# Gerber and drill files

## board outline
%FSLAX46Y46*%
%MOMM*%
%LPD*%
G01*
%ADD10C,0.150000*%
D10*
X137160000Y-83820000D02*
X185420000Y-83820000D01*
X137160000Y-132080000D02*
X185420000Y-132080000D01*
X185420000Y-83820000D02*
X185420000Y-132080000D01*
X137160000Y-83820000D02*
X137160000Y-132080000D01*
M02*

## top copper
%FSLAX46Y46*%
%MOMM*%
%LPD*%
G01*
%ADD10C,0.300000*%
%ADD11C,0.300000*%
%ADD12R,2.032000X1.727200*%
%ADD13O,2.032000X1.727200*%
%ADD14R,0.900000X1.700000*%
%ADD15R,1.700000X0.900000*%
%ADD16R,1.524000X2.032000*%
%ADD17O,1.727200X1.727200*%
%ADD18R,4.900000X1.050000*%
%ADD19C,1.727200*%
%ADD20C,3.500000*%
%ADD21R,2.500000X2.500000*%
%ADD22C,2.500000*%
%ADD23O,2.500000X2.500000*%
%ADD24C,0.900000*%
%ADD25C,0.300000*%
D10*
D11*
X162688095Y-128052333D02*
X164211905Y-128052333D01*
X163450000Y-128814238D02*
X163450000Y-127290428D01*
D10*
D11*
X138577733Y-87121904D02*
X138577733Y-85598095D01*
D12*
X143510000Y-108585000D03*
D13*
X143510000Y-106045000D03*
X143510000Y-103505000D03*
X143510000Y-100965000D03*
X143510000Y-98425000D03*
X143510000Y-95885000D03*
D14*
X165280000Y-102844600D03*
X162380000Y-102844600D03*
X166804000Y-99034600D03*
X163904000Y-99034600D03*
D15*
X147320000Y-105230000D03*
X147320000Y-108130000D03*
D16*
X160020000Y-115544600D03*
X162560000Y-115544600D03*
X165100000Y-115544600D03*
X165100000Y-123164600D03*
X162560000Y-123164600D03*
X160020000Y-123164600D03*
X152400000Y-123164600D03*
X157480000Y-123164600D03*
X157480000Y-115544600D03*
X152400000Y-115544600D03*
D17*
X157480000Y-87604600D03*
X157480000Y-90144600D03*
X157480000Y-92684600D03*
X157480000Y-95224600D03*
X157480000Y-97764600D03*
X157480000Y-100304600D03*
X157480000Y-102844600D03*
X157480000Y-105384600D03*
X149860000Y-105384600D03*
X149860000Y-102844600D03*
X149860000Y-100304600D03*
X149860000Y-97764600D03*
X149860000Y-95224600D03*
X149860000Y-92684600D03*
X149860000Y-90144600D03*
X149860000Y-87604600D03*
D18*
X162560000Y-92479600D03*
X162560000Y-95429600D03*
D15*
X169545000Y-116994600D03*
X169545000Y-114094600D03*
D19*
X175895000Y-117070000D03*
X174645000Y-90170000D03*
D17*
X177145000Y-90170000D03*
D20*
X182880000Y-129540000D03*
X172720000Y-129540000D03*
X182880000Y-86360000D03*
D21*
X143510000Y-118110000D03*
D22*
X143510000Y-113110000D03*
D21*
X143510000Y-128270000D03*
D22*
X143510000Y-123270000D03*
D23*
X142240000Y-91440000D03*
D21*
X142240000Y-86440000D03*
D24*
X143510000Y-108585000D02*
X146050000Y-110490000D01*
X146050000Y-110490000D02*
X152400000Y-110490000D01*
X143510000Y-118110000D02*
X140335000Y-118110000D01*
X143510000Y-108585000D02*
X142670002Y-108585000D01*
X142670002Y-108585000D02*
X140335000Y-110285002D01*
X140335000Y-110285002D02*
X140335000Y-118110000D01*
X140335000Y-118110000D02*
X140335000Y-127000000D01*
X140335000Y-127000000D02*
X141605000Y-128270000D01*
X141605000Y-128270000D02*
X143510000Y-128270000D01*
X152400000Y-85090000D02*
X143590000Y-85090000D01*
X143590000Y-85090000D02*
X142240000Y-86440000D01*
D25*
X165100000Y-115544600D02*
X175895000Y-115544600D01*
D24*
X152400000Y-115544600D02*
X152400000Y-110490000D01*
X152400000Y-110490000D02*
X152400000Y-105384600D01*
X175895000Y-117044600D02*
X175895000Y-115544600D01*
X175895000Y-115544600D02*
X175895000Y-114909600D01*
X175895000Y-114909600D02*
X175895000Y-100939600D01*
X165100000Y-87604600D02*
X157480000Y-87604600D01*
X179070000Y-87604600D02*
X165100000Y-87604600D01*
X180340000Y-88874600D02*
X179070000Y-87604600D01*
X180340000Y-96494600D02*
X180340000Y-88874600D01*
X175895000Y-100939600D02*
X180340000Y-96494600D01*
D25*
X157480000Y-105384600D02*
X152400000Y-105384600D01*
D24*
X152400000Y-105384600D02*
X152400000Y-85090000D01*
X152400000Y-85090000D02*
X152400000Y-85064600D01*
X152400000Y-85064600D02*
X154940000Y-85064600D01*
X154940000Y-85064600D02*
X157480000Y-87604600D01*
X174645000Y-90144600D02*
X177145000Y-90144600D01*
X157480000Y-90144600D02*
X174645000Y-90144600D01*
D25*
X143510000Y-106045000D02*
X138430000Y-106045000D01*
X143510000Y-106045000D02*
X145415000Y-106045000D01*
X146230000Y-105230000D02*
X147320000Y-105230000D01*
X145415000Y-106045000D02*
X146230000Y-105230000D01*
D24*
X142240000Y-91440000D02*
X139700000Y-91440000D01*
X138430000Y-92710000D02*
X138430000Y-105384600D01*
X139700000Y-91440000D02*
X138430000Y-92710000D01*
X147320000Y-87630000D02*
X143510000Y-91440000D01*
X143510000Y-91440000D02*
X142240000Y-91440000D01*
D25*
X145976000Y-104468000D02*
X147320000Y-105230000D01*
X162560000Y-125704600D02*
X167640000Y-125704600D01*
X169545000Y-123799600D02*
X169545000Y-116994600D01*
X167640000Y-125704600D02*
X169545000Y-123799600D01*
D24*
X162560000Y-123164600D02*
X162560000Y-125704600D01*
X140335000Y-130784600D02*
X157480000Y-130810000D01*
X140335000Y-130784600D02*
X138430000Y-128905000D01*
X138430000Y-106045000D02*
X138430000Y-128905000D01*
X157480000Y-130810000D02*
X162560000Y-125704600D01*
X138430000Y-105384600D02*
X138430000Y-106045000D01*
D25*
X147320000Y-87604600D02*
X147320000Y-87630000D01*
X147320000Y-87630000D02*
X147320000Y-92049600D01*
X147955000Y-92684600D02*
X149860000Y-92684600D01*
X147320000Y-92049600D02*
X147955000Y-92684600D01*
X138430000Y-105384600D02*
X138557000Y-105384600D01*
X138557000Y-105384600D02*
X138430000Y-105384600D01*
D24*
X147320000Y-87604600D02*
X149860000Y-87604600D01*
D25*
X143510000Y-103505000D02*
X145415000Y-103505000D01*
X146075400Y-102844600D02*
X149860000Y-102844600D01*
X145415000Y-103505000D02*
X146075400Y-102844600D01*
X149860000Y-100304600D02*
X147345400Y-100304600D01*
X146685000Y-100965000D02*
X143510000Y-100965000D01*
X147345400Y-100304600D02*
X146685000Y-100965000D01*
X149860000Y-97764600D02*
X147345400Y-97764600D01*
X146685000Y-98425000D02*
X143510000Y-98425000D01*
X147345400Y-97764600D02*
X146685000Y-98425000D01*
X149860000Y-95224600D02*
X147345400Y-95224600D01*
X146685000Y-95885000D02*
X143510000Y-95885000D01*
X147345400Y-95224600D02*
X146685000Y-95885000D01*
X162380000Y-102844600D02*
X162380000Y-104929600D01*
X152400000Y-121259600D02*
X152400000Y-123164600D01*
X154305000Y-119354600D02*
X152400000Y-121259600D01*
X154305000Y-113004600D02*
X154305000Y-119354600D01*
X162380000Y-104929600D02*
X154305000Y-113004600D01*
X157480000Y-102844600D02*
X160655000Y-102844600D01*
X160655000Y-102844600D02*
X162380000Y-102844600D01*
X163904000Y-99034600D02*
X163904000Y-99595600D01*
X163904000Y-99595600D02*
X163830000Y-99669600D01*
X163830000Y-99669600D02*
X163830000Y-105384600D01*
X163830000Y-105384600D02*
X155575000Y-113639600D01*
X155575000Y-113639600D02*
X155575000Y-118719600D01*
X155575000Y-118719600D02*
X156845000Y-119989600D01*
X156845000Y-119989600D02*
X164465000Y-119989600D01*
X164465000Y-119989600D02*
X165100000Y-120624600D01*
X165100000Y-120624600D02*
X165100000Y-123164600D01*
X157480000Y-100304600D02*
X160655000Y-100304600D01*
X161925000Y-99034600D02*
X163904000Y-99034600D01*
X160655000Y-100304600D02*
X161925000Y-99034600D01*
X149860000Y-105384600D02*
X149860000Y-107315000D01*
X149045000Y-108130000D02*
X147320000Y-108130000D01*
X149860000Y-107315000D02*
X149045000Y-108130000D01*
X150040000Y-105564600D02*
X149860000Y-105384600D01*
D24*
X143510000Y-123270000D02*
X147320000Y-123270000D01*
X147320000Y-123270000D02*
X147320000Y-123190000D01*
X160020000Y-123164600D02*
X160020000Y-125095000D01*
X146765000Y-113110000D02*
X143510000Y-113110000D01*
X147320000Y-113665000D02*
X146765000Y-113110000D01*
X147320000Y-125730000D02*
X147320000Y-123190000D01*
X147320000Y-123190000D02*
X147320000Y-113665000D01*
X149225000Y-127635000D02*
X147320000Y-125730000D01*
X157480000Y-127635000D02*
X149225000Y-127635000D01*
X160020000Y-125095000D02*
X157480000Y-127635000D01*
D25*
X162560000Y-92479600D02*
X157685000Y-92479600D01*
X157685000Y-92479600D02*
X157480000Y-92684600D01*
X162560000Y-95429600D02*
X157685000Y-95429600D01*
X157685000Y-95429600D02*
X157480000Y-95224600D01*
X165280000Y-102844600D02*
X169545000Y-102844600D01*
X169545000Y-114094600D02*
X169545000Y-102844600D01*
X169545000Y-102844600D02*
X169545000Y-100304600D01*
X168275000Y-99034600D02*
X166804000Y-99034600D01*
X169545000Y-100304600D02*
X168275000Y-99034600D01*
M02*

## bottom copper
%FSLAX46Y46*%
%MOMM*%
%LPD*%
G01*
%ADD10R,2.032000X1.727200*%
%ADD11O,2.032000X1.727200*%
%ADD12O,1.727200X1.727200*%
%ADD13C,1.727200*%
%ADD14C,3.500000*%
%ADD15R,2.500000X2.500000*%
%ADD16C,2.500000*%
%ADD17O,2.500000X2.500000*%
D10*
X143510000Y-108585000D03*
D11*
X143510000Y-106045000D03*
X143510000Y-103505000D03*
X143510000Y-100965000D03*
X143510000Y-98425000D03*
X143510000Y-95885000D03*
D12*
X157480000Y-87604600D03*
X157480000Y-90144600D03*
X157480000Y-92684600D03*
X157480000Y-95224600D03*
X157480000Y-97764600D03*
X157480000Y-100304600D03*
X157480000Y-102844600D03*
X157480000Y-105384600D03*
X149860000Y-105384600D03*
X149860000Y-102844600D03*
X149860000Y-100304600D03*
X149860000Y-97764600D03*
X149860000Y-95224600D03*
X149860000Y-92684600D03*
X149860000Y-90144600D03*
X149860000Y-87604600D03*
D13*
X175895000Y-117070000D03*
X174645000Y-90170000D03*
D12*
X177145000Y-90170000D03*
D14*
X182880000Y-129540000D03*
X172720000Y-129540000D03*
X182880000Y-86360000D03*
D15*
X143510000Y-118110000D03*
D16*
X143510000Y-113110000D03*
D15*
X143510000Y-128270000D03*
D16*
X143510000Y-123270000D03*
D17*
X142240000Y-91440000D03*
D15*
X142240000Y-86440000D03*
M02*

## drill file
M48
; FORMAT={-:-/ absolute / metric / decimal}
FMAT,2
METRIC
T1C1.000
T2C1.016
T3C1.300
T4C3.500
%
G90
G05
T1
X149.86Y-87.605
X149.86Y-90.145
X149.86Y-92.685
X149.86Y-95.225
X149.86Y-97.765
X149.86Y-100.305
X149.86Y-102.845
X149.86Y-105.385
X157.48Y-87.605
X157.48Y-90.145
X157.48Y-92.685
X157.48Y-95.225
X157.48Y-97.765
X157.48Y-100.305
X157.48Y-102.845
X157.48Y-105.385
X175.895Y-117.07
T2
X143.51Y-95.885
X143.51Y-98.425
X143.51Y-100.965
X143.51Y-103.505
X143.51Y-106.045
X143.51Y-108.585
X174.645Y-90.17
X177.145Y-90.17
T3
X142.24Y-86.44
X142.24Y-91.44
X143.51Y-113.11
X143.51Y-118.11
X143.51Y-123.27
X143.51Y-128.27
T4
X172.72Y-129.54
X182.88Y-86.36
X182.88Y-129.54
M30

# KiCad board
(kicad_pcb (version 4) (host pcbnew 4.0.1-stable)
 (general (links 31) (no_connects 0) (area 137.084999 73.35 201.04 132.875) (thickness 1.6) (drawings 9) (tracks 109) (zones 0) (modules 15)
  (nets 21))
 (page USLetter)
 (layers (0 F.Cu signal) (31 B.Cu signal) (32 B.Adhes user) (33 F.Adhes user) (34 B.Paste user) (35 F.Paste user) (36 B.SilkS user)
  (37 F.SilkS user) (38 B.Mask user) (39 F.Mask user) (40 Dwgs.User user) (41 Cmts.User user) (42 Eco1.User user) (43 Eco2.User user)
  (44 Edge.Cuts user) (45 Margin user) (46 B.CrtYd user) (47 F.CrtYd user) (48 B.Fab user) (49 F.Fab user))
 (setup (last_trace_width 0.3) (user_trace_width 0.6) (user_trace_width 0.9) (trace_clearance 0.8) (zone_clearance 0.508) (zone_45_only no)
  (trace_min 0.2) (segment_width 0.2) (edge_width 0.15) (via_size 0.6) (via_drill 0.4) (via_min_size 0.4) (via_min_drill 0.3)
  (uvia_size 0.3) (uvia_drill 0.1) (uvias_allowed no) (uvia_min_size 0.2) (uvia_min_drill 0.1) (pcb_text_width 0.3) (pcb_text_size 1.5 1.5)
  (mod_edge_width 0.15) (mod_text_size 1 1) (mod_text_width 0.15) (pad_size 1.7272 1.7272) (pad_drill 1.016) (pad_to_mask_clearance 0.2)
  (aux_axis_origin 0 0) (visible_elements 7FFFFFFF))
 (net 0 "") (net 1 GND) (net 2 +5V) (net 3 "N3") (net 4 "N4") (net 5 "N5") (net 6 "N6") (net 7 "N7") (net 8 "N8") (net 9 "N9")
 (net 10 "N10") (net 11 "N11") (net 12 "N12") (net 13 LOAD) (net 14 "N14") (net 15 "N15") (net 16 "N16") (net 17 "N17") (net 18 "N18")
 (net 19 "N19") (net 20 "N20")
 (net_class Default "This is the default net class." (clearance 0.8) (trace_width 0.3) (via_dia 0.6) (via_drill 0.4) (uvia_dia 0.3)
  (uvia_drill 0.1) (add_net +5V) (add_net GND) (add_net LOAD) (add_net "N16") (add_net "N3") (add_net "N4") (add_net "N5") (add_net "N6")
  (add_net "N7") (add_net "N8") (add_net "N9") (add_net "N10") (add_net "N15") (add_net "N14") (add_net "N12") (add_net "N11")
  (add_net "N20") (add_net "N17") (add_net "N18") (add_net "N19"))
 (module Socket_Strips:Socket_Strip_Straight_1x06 (layer B.Cu) (at 143.51 108.585 90)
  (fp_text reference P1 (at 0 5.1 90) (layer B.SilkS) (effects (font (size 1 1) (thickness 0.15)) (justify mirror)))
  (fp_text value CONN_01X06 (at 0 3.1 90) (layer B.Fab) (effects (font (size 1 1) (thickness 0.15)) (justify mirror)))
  (pad 1 thru_hole rect (at 0 0 90) (size 1.7272 2.032) (drill 1.016) (layers *.Cu *.Mask B.SilkS) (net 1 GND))
  (pad 2 thru_hole oval (at 2.54 0 90) (size 1.7272 2.032) (drill 1.016) (layers *.Cu *.Mask B.SilkS) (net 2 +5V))
  (pad 3 thru_hole oval (at 5.08 0 90) (size 1.7272 2.032) (drill 1.016) (layers *.Cu *.Mask B.SilkS) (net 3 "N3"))
  (pad 4 thru_hole oval (at 7.62 0 90) (size 1.7272 2.032) (drill 1.016) (layers *.Cu *.Mask B.SilkS) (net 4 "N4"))
  (pad 5 thru_hole oval (at 10.16 0 90) (size 1.7272 2.032) (drill 1.016) (layers *.Cu *.Mask B.SilkS) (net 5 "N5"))
  (pad 6 thru_hole oval (at 12.7 0 90) (size 1.7272 2.032) (drill 1.016) (layers *.Cu *.Mask B.SilkS) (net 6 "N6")))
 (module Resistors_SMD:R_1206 (layer F.Cu) (at 163.83 102.8446 180)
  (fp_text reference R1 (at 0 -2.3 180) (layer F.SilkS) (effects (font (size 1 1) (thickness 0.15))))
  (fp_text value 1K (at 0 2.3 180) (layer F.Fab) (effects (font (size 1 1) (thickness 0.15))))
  (pad 1 smd rect (at -1.45 0 180) (size 0.9 1.7) (layers F.Cu F.Paste F.Mask) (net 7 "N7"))
  (pad 2 smd rect (at 1.45 0 180) (size 0.9 1.7) (layers F.Cu F.Paste F.Mask) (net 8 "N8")))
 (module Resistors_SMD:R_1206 (layer F.Cu) (at 165.354 99.0346 180)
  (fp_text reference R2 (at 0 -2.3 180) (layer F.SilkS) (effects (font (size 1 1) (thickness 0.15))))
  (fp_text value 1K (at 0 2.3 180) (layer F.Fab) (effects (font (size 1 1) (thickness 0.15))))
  (pad 1 smd rect (at -1.45 0 180) (size 0.9 1.7) (layers F.Cu F.Paste F.Mask) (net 7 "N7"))
  (pad 2 smd rect (at 1.45 0 180) (size 0.9 1.7) (layers F.Cu F.Paste F.Mask) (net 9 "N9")))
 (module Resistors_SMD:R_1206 (layer F.Cu) (at 147.32 106.68 270)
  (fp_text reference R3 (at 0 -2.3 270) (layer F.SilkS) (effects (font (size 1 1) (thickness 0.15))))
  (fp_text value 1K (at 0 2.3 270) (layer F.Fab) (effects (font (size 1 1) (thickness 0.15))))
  (pad 1 smd rect (at -1.45 0 270) (size 0.9 1.7) (layers F.Cu F.Paste F.Mask) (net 2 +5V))
  (pad 2 smd rect (at 1.45 0 270) (size 0.9 1.7) (layers F.Cu F.Paste F.Mask) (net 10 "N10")))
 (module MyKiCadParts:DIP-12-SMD (layer F.Cu) (at 152.4 123.1646)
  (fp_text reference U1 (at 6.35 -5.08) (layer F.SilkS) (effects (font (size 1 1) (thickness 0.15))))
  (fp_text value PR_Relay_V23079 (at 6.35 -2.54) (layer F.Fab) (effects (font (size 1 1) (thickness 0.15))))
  (pad 9 smd rect (at 7.62 -7.62) (size 1.524 2.032) (layers F.Cu F.Paste F.Mask) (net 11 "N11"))
  (pad 8 smd rect (at 10.16 -7.62) (size 1.524 2.032) (layers F.Cu F.Paste F.Mask) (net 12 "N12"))
  (pad 7 smd rect (at 12.7 -7.62) (size 1.524 2.032) (layers F.Cu F.Paste F.Mask) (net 1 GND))
  (pad 6 smd rect (at 12.7 0) (size 1.524 2.032) (layers F.Cu F.Paste F.Mask) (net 9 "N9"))
  (pad 5 smd rect (at 10.16 0) (size 1.524 2.032) (layers F.Cu F.Paste F.Mask) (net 2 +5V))
  (pad 4 smd rect (at 7.62 0) (size 1.524 2.032) (layers F.Cu F.Paste F.Mask) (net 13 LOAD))
  (pad 1 smd rect (at 0 0) (size 1.524 2.032) (layers F.Cu F.Paste F.Mask) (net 8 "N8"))
  (pad 3 smd rect (at 5.08 0) (size 1.524 2.032) (layers F.Cu F.Paste F.Mask) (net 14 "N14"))
  (pad 10 smd rect (at 5.08 -7.62) (size 1.524 2.032) (layers F.Cu F.Paste F.Mask) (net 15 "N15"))
  (pad 12 smd rect (at 0 -7.62) (size 1.524 2.032) (layers F.Cu F.Paste F.Mask) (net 1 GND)))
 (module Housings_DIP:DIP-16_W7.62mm (layer B.Cu) (at 157.48 87.6046 180)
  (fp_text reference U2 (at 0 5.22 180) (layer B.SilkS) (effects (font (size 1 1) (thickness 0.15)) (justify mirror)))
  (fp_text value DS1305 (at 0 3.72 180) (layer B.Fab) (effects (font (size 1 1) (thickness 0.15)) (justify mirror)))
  (pad 1 thru_hole oval (at 0 0 180) (size 1.7272 1.7272) (drill 1) (layers *.Cu *.Mask B.SilkS) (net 1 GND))
  (pad 2 thru_hole oval (at 0 -2.54 180) (size 1.7272 1.7272) (drill 1) (layers *.Cu *.Mask B.SilkS) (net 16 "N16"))
  (pad 3 thru_hole oval (at 0 -5.08 180) (size 1.7272 1.7272) (drill 1) (layers *.Cu *.Mask B.SilkS) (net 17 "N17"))
  (pad 4 thru_hole oval (at 0 -7.62 180) (size 1.7272 1.7272) (drill 1) (layers *.Cu *.Mask B.SilkS) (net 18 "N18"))
  (pad 5 thru_hole oval (at 0 -10.16 180) (size 1.7272 1.7272) (drill 1) (layers *.Cu *.Mask B.SilkS) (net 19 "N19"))
  (pad 6 thru_hole oval (at 0 -12.7 180) (size 1.7272 1.7272) (drill 1) (layers *.Cu *.Mask B.SilkS) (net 9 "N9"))
  (pad 7 thru_hole oval (at 0 -15.24 180) (size 1.7272 1.7272) (drill 1) (layers *.Cu *.Mask B.SilkS) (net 8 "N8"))
  (pad 8 thru_hole oval (at 0 -17.78 180) (size 1.7272 1.7272) (drill 1) (layers *.Cu *.Mask B.SilkS) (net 1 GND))
  (pad 9 thru_hole oval (at 7.62 -17.78 180) (size 1.7272 1.7272) (drill 1) (layers *.Cu *.Mask B.SilkS) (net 10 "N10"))
  (pad 10 thru_hole oval (at 7.62 -15.24 180) (size 1.7272 1.7272) (drill 1) (layers *.Cu *.Mask B.SilkS) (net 3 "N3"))
  (pad 11 thru_hole oval (at 7.62 -12.7 180) (size 1.7272 1.7272) (drill 1) (layers *.Cu *.Mask B.SilkS) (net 4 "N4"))
  (pad 12 thru_hole oval (at 7.62 -10.16 180) (size 1.7272 1.7272) (drill 1) (layers *.Cu *.Mask B.SilkS) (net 5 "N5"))
  (pad 13 thru_hole oval (at 7.62 -7.62 180) (size 1.7272 1.7272) (drill 1) (layers *.Cu *.Mask B.SilkS) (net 6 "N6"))
  (pad 14 thru_hole oval (at 7.62 -5.08 180) (size 1.7272 1.7272) (drill 1) (layers *.Cu *.Mask B.SilkS) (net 2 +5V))
  (pad 15 thru_hole oval (at 7.62 -2.54 180) (size 1.7272 1.7272) (drill 1) (layers *.Cu *.Mask B.SilkS) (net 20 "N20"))
  (pad 16 thru_hole oval (at 7.62 0 180) (size 1.7272 1.7272) (drill 1) (layers *.Cu *.Mask B.SilkS) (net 2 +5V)))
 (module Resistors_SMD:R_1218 (layer F.Cu) (at 162.56 93.9546 270)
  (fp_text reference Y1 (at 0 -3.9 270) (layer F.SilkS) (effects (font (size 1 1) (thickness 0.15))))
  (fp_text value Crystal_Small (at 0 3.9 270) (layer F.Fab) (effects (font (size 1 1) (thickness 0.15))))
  (pad 1 smd rect (at -1.475 0 270) (size 1.05 4.9) (layers F.Cu F.Paste F.Mask) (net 17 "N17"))
  (pad 2 smd rect (at 1.475 0 270) (size 1.05 4.9) (layers F.Cu F.Paste F.Mask) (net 18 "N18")))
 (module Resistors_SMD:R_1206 (layer F.Cu) (at 169.545 115.5446 90)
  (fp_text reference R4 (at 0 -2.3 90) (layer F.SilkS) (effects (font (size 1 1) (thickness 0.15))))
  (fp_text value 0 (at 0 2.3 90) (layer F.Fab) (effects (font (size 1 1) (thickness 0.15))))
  (pad 1 smd rect (at -1.45 0 90) (size 0.9 1.7) (layers F.Cu F.Paste F.Mask) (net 2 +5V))
  (pad 2 smd rect (at 1.45 0 90) (size 0.9 1.7) (layers F.Cu F.Paste F.Mask) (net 7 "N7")))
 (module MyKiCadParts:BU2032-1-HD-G (layer B.Cu) (at 175.895 90.17 270)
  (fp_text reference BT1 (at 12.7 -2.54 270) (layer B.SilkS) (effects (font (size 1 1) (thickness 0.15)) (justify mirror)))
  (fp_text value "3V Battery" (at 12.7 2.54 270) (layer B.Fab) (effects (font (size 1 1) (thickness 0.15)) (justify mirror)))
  (pad 2 thru_hole circle (at 26.9 0 270) (size 1.7272 1.7272) (drill 1) (layers *.Cu *.Mask B.SilkS) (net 1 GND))
  (pad 1 thru_hole circle (at 0 1.25 270) (size 1.7272 1.7272) (drill 1.016) (layers *.Cu *.Mask B.SilkS) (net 16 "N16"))
  (pad 1 thru_hole oval (at 0 -1.25 270) (size 1.7272 1.7272) (drill 1.016) (layers *.Cu *.Mask B.SilkS) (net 16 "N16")))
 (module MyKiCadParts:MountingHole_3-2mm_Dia (layer F.Cu) (at 182.88 129.54)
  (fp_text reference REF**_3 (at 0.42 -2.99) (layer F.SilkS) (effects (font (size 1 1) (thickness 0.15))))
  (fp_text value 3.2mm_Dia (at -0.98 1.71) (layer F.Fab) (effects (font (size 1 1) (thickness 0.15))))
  (pad 1 thru_hole circle (at 0 0) (size 3.5 3.5) (drill 3.5)))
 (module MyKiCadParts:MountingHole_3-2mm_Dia (layer F.Cu) (at 172.72 129.54)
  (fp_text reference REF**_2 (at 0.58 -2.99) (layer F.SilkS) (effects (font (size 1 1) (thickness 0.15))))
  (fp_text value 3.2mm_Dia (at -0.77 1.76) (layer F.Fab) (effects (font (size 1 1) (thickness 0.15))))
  (pad 1 thru_hole circle (at 0 0) (size 3.5 3.5) (drill 3.5)))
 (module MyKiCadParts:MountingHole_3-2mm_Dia (layer F.Cu) (at 182.88 86.36)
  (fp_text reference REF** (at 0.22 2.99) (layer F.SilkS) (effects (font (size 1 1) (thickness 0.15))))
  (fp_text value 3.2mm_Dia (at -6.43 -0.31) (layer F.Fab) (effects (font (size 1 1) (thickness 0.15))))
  (pad 1 thru_hole circle (at 0 0) (size 3.5 3.5) (drill 3.5)))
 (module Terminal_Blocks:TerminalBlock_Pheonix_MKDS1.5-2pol (layer B.Cu) (at 143.51 118.11 90)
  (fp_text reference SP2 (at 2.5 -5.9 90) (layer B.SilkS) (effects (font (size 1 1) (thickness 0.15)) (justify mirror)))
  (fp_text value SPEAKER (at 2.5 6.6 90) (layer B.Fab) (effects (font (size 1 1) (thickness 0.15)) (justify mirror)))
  (pad 1 thru_hole rect (at 0 0 90) (size 2.5 2.5) (drill 1.3) (layers *.Cu *.Mask B.SilkS) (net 1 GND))
  (pad 2 thru_hole circle (at 5 0 90) (size 2.5 2.5) (drill 1.3) (layers *.Cu *.Mask B.SilkS) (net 13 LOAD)))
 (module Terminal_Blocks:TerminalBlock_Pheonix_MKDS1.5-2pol (layer B.Cu) (at 143.51 128.27 90)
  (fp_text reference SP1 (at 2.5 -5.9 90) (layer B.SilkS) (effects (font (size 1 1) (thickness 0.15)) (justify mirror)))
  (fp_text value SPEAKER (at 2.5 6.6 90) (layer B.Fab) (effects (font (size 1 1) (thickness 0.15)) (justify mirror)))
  (pad 1 thru_hole rect (at 0 0 90) (size 2.5 2.5) (drill 1.3) (layers *.Cu *.Mask B.SilkS) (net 1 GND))
  (pad 2 thru_hole circle (at 5 0 90) (size 2.5 2.5) (drill 1.3) (layers *.Cu *.Mask B.SilkS) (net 13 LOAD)))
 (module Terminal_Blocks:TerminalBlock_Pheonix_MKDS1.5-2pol (layer B.Cu) (at 142.24 91.44 90)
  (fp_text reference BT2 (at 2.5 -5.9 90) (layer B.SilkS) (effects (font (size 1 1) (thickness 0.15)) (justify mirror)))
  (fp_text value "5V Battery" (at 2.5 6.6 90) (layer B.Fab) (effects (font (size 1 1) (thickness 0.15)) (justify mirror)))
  (pad 1 thru_hole oval (at 0 0 90) (size 2.5 2.5) (drill 1.3) (layers *.Cu *.Mask B.SilkS) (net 2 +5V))
  (pad 2 thru_hole rect (at 5 0 90) (size 2.5 2.5) (drill 1.3) (layers *.Cu *.Mask B.SilkS) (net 1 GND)))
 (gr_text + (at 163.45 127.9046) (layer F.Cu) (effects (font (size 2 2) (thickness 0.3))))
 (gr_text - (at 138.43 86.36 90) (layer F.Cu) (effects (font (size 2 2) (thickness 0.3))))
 (gr_line (start 137.16 83.82) (end 185.42 83.82) (angle 90) (layer Edge.Cuts) (width 0.15))
 (gr_line (start 137.16 132.08) (end 185.42 132.08) (angle 90) (layer Edge.Cuts) (width 0.15))
 (gr_line (start 185.42 83.82) (end 185.42 132.08) (angle 90) (layer Edge.Cuts) (width 0.15))
 (gr_line (start 137.16 83.82) (end 137.16 132.08) (angle 90) (layer Edge.Cuts) (width 0.15))
 (segment (start 143.51 108.585) (end 146.05 110.49) (width 0.9) (layer F.Cu) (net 1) (status 10))
 (segment (start 146.05 110.49) (end 152.4 110.49) (width 0.9) (layer F.Cu) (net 1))
 (segment (start 143.51 118.11) (end 140.335 118.11) (width 0.9) (layer F.Cu) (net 1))
 (segment (start 143.51 108.585) (end 142.670002 108.585) (width 0.9) (layer F.Cu) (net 1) (status 30))
 (segment (start 142.670002 108.585) (end 140.335 110.285002) (width 0.9) (layer F.Cu) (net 1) (status 10))
 (segment (start 140.335 110.285002) (end 140.335 118.11) (width 0.9) (layer F.Cu) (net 1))
 (segment (start 140.335 118.11) (end 140.335 127) (width 0.9) (layer F.Cu) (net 1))
 (segment (start 140.335 127) (end 141.605 128.27) (width 0.9) (layer F.Cu) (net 1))
 (segment (start 141.605 128.27) (end 143.51 128.27) (width 0.9) (layer F.Cu) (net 1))
 (segment (start 152.4 85.09) (end 143.59 85.09) (width 0.9) (layer F.Cu) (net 1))
 (segment (start 143.59 85.09) (end 142.24 86.44) (width 0.9) (layer F.Cu) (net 1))
 (segment (start 165.1 115.5446) (end 175.895 115.5446) (width 0.3) (layer F.Cu) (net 1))
 (segment (start 152.4 115.5446) (end 152.4 110.49) (width 0.9) (layer F.Cu) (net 1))
 (segment (start 152.4 110.49) (end 152.4 105.3846) (width 0.9) (layer F.Cu) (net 1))
 (segment (start 175.895 117.0446) (end 175.895 115.5446) (width 0.9) (layer F.Cu) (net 1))
 (segment (start 175.895 115.5446) (end 175.895 114.9096) (width 0.9) (layer F.Cu) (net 1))
 (segment (start 175.895 114.9096) (end 175.895 100.9396) (width 0.9) (layer F.Cu) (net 1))
 (segment (start 165.1 87.6046) (end 157.48 87.6046) (width 0.9) (layer F.Cu) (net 1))
 (segment (start 179.07 87.6046) (end 165.1 87.6046) (width 0.9) (layer F.Cu) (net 1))
 (segment (start 180.34 88.8746) (end 179.07 87.6046) (width 0.9) (layer F.Cu) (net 1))
 (segment (start 180.34 96.4946) (end 180.34 88.8746) (width 0.9) (layer F.Cu) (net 1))
 (segment (start 175.895 100.9396) (end 180.34 96.4946) (width 0.9) (layer F.Cu) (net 1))
 (segment (start 157.48 105.3846) (end 152.4 105.3846) (width 0.3) (layer F.Cu) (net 1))
 (segment (start 152.4 105.3846) (end 152.4 85.09) (width 0.9) (layer F.Cu) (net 1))
 (segment (start 152.4 85.09) (end 152.4 85.0646) (width 0.9) (layer F.Cu) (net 1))
 (segment (start 152.4 85.0646) (end 154.94 85.0646) (width 0.9) (layer F.Cu) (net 1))
 (segment (start 154.94 85.0646) (end 157.48 87.6046) (width 0.9) (layer F.Cu) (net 1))
 (segment (start 174.645 90.1446) (end 177.145 90.1446) (width 0.9) (layer F.Cu) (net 16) (status 30))
 (segment (start 157.48 90.1446) (end 174.645 90.1446) (width 0.9) (layer F.Cu) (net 16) (status 20))
 (segment (start 143.51 106.045) (end 138.43 106.045) (width 0.3) (layer F.Cu) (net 2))
 (segment (start 143.51 106.045) (end 145.415 106.045) (width 0.3) (layer F.Cu) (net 2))
 (segment (start 146.23 105.23) (end 147.32 105.23) (width 0.3) (layer F.Cu) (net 2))
 (segment (start 145.415 106.045) (end 146.23 105.23) (width 0.3) (layer F.Cu) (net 2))
 (segment (start 142.24 91.44) (end 139.7 91.44) (width 0.9) (layer F.Cu) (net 2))
 (segment (start 138.43 92.71) (end 138.43 105.3846) (width 0.9) (layer F.Cu) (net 2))
 (segment (start 139.7 91.44) (end 138.43 92.71) (width 0.9) (layer F.Cu) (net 2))
 (segment (start 147.32 87.63) (end 143.51 91.44) (width 0.9) (layer F.Cu) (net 2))
 (segment (start 143.51 91.44) (end 142.24 91.44) (width 0.9) (layer F.Cu) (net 2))
 (segment (start 145.976 104.468) (end 147.32 105.23) (width 0.3) (layer F.Cu) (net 2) (status 20))
 (segment (start 162.56 125.7046) (end 167.64 125.7046) (width 0.3) (layer F.Cu) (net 2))
 (segment (start 169.545 123.7996) (end 169.545 116.9946) (width 0.3) (layer F.Cu) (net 2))
 (segment (start 167.64 125.7046) (end 169.545 123.7996) (width 0.3) (layer F.Cu) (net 2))
 (segment (start 162.56 123.1646) (end 162.56 125.7046) (width 0.9) (layer F.Cu) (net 2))
 (segment (start 140.335 130.7846) (end 157.48 130.81) (width 0.9) (layer F.Cu) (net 2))
 (segment (start 140.335 130.7846) (end 138.43 128.905) (width 0.9) (layer F.Cu) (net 2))
 (segment (start 138.43 106.045) (end 138.43 128.905) (width 0.9) (layer F.Cu) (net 2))
 (segment (start 157.48 130.81) (end 162.56 125.7046) (width 0.9) (layer F.Cu) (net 2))
 (segment (start 138.43 105.3846) (end 138.43 106.045) (width 0.9) (layer F.Cu) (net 2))
 (segment (start 147.32 87.6046) (end 147.32 87.63) (width 0.3) (layer F.Cu) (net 2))
 (segment (start 147.32 87.63) (end 147.32 92.0496) (width 0.3) (layer F.Cu) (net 2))
 (segment (start 147.955 92.6846) (end 149.86 92.6846) (width 0.3) (layer F.Cu) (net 2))
 (segment (start 147.32 92.0496) (end 147.955 92.6846) (width 0.3) (layer F.Cu) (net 2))
 (segment (start 138.43 105.3846) (end 138.557 105.3846) (width 0.3) (layer F.Cu) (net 2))
 (segment (start 138.557 105.3846) (end 138.43 105.3846) (width 0.3) (layer F.Cu) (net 2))
 (segment (start 147.32 87.6046) (end 149.86 87.6046) (width 0.9) (layer F.Cu) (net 2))
 (segment (start 143.51 103.505) (end 145.415 103.505) (width 0.3) (layer F.Cu) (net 3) (status 400000))
 (segment (start 146.0754 102.8446) (end 149.86 102.8446) (width 0.3) (layer F.Cu) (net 3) (status 800000))
 (segment (start 145.415 103.505) (end 146.0754 102.8446) (width 0.3) (layer F.Cu) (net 3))
 (segment (start 149.86 100.3046) (end 147.3454 100.3046) (width 0.3) (layer F.Cu) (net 4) (status 400000))
 (segment (start 146.685 100.965) (end 143.51 100.965) (width 0.3) (layer F.Cu) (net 4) (status 800000))
 (segment (start 147.3454 100.3046) (end 146.685 100.965) (width 0.3) (layer F.Cu) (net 4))
 (segment (start 149.86 97.7646) (end 147.3454 97.7646) (width 0.3) (layer F.Cu) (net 5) (status 400000))
 (segment (start 146.685 98.425) (end 143.51 98.425) (width 0.3) (layer F.Cu) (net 5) (status 800000))
 (segment (start 147.3454 97.7646) (end 146.685 98.425) (width 0.3) (layer F.Cu) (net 5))
 (segment (start 149.86 95.2246) (end 147.3454 95.2246) (width 0.3) (layer F.Cu) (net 6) (status 400000))
 (segment (start 146.685 95.885) (end 143.51 95.885) (width 0.3) (layer F.Cu) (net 6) (status 800000))
 (segment (start 147.3454 95.2246) (end 146.685 95.885) (width 0.3) (layer F.Cu) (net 6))
 (segment (start 162.38 102.8446) (end 162.38 104.9296) (width 0.3) (layer F.Cu) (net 8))
 (segment (start 152.4 121.2596) (end 152.4 123.1646) (width 0.3) (layer F.Cu) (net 8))
 (segment (start 154.305 119.3546) (end 152.4 121.2596) (width 0.3) (layer F.Cu) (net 8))
 (segment (start 154.305 113.0046) (end 154.305 119.3546) (width 0.3) (layer F.Cu) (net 8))
 (segment (start 162.38 104.9296) (end 154.305 113.0046) (width 0.3) (layer F.Cu) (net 8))
 (segment (start 157.48 102.8446) (end 160.655 102.8446) (width 0.3) (layer F.Cu) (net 8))
 (segment (start 160.655 102.8446) (end 162.38 102.8446) (width 0.3) (layer F.Cu) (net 8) (status 20))
 (segment (start 163.904 99.0346) (end 163.904 99.5956) (width 0.3) (layer F.Cu) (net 9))
 (segment (start 163.904 99.5956) (end 163.83 99.6696) (width 0.3) (layer F.Cu) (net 9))
 (segment (start 163.83 99.6696) (end 163.83 105.3846) (width 0.3) (layer F.Cu) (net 9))
 (segment (start 163.83 105.3846) (end 155.575 113.6396) (width 0.3) (layer F.Cu) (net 9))
 (segment (start 155.575 113.6396) (end 155.575 118.7196) (width 0.3) (layer F.Cu) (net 9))
 (segment (start 155.575 118.7196) (end 156.845 119.9896) (width 0.3) (layer F.Cu) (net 9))
 (segment (start 156.845 119.9896) (end 164.465 119.9896) (width 0.3) (layer F.Cu) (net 9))
 (segment (start 164.465 119.9896) (end 165.1 120.6246) (width 0.3) (layer F.Cu) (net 9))
 (segment (start 165.1 120.6246) (end 165.1 123.1646) (width 0.3) (layer F.Cu) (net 9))
 (segment (start 157.48 100.3046) (end 160.655 100.3046) (width 0.3) (layer F.Cu) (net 9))
 (segment (start 161.925 99.0346) (end 163.904 99.0346) (width 0.3) (layer F.Cu) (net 9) (status 20))
 (segment (start 160.655 100.3046) (end 161.925 99.0346) (width 0.3) (layer F.Cu) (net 9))
 (segment (start 149.86 105.3846) (end 149.86 107.315) (width 0.3) (layer F.Cu) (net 10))
 (segment (start 149.045 108.13) (end 147.32 108.13) (width 0.3) (layer F.Cu) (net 10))
 (segment (start 149.86 107.315) (end 149.045 108.13) (width 0.3) (layer F.Cu) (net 10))
 (segment (start 150.04 105.5646) (end 149.86 105.3846) (width 0.3) (layer F.Cu) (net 10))
 (segment (start 143.51 123.27) (end 147.32 123.27) (width 0.9) (layer F.Cu) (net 13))
 (segment (start 147.32 123.27) (end 147.32 123.19) (width 0.9) (layer F.Cu) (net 13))
 (segment (start 160.02 123.1646) (end 160.02 125.095) (width 0.9) (layer F.Cu) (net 13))
 (segment (start 146.765 113.11) (end 143.51 113.11) (width 0.9) (layer F.Cu) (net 13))
 (segment (start 147.32 113.665) (end 146.765 113.11) (width 0.9) (layer F.Cu) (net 13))
 (segment (start 147.32 125.73) (end 147.32 123.19) (width 0.9) (layer F.Cu) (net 13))
 (segment (start 147.32 123.19) (end 147.32 113.665) (width 0.9) (layer F.Cu) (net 13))
 (segment (start 149.225 127.635) (end 147.32 125.73) (width 0.9) (layer F.Cu) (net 13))
 (segment (start 157.48 127.635) (end 149.225 127.635) (width 0.9) (layer F.Cu) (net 13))
 (segment (start 160.02 125.095) (end 157.48 127.635) (width 0.9) (layer F.Cu) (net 13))
 (segment (start 162.56 92.4796) (end 157.685 92.4796) (width 0.3) (layer F.Cu) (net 17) (status 10))
 (segment (start 157.685 92.4796) (end 157.48 92.6846) (width 0.3) (layer F.Cu) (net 17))
 (segment (start 162.56 95.4296) (end 157.685 95.4296) (width 0.3) (layer F.Cu) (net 18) (status 10))
 (segment (start 157.685 95.4296) (end 157.48 95.2246) (width 0.3) (layer F.Cu) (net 18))
 (segment (start 165.28 102.8446) (end 169.545 102.8446) (width 0.3) (layer F.Cu) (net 7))
 (segment (start 169.545 114.0946) (end 169.545 102.8446) (width 0.3) (layer F.Cu) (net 7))
 (segment (start 169.545 102.8446) (end 169.545 100.3046) (width 0.3) (layer F.Cu) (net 7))
 (segment (start 168.275 99.0346) (end 166.804 99.0346) (width 0.3) (layer F.Cu) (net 7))
 (segment (start 169.545 100.3046) (end 168.275 99.0346) (width 0.3) (layer F.Cu) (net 7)))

